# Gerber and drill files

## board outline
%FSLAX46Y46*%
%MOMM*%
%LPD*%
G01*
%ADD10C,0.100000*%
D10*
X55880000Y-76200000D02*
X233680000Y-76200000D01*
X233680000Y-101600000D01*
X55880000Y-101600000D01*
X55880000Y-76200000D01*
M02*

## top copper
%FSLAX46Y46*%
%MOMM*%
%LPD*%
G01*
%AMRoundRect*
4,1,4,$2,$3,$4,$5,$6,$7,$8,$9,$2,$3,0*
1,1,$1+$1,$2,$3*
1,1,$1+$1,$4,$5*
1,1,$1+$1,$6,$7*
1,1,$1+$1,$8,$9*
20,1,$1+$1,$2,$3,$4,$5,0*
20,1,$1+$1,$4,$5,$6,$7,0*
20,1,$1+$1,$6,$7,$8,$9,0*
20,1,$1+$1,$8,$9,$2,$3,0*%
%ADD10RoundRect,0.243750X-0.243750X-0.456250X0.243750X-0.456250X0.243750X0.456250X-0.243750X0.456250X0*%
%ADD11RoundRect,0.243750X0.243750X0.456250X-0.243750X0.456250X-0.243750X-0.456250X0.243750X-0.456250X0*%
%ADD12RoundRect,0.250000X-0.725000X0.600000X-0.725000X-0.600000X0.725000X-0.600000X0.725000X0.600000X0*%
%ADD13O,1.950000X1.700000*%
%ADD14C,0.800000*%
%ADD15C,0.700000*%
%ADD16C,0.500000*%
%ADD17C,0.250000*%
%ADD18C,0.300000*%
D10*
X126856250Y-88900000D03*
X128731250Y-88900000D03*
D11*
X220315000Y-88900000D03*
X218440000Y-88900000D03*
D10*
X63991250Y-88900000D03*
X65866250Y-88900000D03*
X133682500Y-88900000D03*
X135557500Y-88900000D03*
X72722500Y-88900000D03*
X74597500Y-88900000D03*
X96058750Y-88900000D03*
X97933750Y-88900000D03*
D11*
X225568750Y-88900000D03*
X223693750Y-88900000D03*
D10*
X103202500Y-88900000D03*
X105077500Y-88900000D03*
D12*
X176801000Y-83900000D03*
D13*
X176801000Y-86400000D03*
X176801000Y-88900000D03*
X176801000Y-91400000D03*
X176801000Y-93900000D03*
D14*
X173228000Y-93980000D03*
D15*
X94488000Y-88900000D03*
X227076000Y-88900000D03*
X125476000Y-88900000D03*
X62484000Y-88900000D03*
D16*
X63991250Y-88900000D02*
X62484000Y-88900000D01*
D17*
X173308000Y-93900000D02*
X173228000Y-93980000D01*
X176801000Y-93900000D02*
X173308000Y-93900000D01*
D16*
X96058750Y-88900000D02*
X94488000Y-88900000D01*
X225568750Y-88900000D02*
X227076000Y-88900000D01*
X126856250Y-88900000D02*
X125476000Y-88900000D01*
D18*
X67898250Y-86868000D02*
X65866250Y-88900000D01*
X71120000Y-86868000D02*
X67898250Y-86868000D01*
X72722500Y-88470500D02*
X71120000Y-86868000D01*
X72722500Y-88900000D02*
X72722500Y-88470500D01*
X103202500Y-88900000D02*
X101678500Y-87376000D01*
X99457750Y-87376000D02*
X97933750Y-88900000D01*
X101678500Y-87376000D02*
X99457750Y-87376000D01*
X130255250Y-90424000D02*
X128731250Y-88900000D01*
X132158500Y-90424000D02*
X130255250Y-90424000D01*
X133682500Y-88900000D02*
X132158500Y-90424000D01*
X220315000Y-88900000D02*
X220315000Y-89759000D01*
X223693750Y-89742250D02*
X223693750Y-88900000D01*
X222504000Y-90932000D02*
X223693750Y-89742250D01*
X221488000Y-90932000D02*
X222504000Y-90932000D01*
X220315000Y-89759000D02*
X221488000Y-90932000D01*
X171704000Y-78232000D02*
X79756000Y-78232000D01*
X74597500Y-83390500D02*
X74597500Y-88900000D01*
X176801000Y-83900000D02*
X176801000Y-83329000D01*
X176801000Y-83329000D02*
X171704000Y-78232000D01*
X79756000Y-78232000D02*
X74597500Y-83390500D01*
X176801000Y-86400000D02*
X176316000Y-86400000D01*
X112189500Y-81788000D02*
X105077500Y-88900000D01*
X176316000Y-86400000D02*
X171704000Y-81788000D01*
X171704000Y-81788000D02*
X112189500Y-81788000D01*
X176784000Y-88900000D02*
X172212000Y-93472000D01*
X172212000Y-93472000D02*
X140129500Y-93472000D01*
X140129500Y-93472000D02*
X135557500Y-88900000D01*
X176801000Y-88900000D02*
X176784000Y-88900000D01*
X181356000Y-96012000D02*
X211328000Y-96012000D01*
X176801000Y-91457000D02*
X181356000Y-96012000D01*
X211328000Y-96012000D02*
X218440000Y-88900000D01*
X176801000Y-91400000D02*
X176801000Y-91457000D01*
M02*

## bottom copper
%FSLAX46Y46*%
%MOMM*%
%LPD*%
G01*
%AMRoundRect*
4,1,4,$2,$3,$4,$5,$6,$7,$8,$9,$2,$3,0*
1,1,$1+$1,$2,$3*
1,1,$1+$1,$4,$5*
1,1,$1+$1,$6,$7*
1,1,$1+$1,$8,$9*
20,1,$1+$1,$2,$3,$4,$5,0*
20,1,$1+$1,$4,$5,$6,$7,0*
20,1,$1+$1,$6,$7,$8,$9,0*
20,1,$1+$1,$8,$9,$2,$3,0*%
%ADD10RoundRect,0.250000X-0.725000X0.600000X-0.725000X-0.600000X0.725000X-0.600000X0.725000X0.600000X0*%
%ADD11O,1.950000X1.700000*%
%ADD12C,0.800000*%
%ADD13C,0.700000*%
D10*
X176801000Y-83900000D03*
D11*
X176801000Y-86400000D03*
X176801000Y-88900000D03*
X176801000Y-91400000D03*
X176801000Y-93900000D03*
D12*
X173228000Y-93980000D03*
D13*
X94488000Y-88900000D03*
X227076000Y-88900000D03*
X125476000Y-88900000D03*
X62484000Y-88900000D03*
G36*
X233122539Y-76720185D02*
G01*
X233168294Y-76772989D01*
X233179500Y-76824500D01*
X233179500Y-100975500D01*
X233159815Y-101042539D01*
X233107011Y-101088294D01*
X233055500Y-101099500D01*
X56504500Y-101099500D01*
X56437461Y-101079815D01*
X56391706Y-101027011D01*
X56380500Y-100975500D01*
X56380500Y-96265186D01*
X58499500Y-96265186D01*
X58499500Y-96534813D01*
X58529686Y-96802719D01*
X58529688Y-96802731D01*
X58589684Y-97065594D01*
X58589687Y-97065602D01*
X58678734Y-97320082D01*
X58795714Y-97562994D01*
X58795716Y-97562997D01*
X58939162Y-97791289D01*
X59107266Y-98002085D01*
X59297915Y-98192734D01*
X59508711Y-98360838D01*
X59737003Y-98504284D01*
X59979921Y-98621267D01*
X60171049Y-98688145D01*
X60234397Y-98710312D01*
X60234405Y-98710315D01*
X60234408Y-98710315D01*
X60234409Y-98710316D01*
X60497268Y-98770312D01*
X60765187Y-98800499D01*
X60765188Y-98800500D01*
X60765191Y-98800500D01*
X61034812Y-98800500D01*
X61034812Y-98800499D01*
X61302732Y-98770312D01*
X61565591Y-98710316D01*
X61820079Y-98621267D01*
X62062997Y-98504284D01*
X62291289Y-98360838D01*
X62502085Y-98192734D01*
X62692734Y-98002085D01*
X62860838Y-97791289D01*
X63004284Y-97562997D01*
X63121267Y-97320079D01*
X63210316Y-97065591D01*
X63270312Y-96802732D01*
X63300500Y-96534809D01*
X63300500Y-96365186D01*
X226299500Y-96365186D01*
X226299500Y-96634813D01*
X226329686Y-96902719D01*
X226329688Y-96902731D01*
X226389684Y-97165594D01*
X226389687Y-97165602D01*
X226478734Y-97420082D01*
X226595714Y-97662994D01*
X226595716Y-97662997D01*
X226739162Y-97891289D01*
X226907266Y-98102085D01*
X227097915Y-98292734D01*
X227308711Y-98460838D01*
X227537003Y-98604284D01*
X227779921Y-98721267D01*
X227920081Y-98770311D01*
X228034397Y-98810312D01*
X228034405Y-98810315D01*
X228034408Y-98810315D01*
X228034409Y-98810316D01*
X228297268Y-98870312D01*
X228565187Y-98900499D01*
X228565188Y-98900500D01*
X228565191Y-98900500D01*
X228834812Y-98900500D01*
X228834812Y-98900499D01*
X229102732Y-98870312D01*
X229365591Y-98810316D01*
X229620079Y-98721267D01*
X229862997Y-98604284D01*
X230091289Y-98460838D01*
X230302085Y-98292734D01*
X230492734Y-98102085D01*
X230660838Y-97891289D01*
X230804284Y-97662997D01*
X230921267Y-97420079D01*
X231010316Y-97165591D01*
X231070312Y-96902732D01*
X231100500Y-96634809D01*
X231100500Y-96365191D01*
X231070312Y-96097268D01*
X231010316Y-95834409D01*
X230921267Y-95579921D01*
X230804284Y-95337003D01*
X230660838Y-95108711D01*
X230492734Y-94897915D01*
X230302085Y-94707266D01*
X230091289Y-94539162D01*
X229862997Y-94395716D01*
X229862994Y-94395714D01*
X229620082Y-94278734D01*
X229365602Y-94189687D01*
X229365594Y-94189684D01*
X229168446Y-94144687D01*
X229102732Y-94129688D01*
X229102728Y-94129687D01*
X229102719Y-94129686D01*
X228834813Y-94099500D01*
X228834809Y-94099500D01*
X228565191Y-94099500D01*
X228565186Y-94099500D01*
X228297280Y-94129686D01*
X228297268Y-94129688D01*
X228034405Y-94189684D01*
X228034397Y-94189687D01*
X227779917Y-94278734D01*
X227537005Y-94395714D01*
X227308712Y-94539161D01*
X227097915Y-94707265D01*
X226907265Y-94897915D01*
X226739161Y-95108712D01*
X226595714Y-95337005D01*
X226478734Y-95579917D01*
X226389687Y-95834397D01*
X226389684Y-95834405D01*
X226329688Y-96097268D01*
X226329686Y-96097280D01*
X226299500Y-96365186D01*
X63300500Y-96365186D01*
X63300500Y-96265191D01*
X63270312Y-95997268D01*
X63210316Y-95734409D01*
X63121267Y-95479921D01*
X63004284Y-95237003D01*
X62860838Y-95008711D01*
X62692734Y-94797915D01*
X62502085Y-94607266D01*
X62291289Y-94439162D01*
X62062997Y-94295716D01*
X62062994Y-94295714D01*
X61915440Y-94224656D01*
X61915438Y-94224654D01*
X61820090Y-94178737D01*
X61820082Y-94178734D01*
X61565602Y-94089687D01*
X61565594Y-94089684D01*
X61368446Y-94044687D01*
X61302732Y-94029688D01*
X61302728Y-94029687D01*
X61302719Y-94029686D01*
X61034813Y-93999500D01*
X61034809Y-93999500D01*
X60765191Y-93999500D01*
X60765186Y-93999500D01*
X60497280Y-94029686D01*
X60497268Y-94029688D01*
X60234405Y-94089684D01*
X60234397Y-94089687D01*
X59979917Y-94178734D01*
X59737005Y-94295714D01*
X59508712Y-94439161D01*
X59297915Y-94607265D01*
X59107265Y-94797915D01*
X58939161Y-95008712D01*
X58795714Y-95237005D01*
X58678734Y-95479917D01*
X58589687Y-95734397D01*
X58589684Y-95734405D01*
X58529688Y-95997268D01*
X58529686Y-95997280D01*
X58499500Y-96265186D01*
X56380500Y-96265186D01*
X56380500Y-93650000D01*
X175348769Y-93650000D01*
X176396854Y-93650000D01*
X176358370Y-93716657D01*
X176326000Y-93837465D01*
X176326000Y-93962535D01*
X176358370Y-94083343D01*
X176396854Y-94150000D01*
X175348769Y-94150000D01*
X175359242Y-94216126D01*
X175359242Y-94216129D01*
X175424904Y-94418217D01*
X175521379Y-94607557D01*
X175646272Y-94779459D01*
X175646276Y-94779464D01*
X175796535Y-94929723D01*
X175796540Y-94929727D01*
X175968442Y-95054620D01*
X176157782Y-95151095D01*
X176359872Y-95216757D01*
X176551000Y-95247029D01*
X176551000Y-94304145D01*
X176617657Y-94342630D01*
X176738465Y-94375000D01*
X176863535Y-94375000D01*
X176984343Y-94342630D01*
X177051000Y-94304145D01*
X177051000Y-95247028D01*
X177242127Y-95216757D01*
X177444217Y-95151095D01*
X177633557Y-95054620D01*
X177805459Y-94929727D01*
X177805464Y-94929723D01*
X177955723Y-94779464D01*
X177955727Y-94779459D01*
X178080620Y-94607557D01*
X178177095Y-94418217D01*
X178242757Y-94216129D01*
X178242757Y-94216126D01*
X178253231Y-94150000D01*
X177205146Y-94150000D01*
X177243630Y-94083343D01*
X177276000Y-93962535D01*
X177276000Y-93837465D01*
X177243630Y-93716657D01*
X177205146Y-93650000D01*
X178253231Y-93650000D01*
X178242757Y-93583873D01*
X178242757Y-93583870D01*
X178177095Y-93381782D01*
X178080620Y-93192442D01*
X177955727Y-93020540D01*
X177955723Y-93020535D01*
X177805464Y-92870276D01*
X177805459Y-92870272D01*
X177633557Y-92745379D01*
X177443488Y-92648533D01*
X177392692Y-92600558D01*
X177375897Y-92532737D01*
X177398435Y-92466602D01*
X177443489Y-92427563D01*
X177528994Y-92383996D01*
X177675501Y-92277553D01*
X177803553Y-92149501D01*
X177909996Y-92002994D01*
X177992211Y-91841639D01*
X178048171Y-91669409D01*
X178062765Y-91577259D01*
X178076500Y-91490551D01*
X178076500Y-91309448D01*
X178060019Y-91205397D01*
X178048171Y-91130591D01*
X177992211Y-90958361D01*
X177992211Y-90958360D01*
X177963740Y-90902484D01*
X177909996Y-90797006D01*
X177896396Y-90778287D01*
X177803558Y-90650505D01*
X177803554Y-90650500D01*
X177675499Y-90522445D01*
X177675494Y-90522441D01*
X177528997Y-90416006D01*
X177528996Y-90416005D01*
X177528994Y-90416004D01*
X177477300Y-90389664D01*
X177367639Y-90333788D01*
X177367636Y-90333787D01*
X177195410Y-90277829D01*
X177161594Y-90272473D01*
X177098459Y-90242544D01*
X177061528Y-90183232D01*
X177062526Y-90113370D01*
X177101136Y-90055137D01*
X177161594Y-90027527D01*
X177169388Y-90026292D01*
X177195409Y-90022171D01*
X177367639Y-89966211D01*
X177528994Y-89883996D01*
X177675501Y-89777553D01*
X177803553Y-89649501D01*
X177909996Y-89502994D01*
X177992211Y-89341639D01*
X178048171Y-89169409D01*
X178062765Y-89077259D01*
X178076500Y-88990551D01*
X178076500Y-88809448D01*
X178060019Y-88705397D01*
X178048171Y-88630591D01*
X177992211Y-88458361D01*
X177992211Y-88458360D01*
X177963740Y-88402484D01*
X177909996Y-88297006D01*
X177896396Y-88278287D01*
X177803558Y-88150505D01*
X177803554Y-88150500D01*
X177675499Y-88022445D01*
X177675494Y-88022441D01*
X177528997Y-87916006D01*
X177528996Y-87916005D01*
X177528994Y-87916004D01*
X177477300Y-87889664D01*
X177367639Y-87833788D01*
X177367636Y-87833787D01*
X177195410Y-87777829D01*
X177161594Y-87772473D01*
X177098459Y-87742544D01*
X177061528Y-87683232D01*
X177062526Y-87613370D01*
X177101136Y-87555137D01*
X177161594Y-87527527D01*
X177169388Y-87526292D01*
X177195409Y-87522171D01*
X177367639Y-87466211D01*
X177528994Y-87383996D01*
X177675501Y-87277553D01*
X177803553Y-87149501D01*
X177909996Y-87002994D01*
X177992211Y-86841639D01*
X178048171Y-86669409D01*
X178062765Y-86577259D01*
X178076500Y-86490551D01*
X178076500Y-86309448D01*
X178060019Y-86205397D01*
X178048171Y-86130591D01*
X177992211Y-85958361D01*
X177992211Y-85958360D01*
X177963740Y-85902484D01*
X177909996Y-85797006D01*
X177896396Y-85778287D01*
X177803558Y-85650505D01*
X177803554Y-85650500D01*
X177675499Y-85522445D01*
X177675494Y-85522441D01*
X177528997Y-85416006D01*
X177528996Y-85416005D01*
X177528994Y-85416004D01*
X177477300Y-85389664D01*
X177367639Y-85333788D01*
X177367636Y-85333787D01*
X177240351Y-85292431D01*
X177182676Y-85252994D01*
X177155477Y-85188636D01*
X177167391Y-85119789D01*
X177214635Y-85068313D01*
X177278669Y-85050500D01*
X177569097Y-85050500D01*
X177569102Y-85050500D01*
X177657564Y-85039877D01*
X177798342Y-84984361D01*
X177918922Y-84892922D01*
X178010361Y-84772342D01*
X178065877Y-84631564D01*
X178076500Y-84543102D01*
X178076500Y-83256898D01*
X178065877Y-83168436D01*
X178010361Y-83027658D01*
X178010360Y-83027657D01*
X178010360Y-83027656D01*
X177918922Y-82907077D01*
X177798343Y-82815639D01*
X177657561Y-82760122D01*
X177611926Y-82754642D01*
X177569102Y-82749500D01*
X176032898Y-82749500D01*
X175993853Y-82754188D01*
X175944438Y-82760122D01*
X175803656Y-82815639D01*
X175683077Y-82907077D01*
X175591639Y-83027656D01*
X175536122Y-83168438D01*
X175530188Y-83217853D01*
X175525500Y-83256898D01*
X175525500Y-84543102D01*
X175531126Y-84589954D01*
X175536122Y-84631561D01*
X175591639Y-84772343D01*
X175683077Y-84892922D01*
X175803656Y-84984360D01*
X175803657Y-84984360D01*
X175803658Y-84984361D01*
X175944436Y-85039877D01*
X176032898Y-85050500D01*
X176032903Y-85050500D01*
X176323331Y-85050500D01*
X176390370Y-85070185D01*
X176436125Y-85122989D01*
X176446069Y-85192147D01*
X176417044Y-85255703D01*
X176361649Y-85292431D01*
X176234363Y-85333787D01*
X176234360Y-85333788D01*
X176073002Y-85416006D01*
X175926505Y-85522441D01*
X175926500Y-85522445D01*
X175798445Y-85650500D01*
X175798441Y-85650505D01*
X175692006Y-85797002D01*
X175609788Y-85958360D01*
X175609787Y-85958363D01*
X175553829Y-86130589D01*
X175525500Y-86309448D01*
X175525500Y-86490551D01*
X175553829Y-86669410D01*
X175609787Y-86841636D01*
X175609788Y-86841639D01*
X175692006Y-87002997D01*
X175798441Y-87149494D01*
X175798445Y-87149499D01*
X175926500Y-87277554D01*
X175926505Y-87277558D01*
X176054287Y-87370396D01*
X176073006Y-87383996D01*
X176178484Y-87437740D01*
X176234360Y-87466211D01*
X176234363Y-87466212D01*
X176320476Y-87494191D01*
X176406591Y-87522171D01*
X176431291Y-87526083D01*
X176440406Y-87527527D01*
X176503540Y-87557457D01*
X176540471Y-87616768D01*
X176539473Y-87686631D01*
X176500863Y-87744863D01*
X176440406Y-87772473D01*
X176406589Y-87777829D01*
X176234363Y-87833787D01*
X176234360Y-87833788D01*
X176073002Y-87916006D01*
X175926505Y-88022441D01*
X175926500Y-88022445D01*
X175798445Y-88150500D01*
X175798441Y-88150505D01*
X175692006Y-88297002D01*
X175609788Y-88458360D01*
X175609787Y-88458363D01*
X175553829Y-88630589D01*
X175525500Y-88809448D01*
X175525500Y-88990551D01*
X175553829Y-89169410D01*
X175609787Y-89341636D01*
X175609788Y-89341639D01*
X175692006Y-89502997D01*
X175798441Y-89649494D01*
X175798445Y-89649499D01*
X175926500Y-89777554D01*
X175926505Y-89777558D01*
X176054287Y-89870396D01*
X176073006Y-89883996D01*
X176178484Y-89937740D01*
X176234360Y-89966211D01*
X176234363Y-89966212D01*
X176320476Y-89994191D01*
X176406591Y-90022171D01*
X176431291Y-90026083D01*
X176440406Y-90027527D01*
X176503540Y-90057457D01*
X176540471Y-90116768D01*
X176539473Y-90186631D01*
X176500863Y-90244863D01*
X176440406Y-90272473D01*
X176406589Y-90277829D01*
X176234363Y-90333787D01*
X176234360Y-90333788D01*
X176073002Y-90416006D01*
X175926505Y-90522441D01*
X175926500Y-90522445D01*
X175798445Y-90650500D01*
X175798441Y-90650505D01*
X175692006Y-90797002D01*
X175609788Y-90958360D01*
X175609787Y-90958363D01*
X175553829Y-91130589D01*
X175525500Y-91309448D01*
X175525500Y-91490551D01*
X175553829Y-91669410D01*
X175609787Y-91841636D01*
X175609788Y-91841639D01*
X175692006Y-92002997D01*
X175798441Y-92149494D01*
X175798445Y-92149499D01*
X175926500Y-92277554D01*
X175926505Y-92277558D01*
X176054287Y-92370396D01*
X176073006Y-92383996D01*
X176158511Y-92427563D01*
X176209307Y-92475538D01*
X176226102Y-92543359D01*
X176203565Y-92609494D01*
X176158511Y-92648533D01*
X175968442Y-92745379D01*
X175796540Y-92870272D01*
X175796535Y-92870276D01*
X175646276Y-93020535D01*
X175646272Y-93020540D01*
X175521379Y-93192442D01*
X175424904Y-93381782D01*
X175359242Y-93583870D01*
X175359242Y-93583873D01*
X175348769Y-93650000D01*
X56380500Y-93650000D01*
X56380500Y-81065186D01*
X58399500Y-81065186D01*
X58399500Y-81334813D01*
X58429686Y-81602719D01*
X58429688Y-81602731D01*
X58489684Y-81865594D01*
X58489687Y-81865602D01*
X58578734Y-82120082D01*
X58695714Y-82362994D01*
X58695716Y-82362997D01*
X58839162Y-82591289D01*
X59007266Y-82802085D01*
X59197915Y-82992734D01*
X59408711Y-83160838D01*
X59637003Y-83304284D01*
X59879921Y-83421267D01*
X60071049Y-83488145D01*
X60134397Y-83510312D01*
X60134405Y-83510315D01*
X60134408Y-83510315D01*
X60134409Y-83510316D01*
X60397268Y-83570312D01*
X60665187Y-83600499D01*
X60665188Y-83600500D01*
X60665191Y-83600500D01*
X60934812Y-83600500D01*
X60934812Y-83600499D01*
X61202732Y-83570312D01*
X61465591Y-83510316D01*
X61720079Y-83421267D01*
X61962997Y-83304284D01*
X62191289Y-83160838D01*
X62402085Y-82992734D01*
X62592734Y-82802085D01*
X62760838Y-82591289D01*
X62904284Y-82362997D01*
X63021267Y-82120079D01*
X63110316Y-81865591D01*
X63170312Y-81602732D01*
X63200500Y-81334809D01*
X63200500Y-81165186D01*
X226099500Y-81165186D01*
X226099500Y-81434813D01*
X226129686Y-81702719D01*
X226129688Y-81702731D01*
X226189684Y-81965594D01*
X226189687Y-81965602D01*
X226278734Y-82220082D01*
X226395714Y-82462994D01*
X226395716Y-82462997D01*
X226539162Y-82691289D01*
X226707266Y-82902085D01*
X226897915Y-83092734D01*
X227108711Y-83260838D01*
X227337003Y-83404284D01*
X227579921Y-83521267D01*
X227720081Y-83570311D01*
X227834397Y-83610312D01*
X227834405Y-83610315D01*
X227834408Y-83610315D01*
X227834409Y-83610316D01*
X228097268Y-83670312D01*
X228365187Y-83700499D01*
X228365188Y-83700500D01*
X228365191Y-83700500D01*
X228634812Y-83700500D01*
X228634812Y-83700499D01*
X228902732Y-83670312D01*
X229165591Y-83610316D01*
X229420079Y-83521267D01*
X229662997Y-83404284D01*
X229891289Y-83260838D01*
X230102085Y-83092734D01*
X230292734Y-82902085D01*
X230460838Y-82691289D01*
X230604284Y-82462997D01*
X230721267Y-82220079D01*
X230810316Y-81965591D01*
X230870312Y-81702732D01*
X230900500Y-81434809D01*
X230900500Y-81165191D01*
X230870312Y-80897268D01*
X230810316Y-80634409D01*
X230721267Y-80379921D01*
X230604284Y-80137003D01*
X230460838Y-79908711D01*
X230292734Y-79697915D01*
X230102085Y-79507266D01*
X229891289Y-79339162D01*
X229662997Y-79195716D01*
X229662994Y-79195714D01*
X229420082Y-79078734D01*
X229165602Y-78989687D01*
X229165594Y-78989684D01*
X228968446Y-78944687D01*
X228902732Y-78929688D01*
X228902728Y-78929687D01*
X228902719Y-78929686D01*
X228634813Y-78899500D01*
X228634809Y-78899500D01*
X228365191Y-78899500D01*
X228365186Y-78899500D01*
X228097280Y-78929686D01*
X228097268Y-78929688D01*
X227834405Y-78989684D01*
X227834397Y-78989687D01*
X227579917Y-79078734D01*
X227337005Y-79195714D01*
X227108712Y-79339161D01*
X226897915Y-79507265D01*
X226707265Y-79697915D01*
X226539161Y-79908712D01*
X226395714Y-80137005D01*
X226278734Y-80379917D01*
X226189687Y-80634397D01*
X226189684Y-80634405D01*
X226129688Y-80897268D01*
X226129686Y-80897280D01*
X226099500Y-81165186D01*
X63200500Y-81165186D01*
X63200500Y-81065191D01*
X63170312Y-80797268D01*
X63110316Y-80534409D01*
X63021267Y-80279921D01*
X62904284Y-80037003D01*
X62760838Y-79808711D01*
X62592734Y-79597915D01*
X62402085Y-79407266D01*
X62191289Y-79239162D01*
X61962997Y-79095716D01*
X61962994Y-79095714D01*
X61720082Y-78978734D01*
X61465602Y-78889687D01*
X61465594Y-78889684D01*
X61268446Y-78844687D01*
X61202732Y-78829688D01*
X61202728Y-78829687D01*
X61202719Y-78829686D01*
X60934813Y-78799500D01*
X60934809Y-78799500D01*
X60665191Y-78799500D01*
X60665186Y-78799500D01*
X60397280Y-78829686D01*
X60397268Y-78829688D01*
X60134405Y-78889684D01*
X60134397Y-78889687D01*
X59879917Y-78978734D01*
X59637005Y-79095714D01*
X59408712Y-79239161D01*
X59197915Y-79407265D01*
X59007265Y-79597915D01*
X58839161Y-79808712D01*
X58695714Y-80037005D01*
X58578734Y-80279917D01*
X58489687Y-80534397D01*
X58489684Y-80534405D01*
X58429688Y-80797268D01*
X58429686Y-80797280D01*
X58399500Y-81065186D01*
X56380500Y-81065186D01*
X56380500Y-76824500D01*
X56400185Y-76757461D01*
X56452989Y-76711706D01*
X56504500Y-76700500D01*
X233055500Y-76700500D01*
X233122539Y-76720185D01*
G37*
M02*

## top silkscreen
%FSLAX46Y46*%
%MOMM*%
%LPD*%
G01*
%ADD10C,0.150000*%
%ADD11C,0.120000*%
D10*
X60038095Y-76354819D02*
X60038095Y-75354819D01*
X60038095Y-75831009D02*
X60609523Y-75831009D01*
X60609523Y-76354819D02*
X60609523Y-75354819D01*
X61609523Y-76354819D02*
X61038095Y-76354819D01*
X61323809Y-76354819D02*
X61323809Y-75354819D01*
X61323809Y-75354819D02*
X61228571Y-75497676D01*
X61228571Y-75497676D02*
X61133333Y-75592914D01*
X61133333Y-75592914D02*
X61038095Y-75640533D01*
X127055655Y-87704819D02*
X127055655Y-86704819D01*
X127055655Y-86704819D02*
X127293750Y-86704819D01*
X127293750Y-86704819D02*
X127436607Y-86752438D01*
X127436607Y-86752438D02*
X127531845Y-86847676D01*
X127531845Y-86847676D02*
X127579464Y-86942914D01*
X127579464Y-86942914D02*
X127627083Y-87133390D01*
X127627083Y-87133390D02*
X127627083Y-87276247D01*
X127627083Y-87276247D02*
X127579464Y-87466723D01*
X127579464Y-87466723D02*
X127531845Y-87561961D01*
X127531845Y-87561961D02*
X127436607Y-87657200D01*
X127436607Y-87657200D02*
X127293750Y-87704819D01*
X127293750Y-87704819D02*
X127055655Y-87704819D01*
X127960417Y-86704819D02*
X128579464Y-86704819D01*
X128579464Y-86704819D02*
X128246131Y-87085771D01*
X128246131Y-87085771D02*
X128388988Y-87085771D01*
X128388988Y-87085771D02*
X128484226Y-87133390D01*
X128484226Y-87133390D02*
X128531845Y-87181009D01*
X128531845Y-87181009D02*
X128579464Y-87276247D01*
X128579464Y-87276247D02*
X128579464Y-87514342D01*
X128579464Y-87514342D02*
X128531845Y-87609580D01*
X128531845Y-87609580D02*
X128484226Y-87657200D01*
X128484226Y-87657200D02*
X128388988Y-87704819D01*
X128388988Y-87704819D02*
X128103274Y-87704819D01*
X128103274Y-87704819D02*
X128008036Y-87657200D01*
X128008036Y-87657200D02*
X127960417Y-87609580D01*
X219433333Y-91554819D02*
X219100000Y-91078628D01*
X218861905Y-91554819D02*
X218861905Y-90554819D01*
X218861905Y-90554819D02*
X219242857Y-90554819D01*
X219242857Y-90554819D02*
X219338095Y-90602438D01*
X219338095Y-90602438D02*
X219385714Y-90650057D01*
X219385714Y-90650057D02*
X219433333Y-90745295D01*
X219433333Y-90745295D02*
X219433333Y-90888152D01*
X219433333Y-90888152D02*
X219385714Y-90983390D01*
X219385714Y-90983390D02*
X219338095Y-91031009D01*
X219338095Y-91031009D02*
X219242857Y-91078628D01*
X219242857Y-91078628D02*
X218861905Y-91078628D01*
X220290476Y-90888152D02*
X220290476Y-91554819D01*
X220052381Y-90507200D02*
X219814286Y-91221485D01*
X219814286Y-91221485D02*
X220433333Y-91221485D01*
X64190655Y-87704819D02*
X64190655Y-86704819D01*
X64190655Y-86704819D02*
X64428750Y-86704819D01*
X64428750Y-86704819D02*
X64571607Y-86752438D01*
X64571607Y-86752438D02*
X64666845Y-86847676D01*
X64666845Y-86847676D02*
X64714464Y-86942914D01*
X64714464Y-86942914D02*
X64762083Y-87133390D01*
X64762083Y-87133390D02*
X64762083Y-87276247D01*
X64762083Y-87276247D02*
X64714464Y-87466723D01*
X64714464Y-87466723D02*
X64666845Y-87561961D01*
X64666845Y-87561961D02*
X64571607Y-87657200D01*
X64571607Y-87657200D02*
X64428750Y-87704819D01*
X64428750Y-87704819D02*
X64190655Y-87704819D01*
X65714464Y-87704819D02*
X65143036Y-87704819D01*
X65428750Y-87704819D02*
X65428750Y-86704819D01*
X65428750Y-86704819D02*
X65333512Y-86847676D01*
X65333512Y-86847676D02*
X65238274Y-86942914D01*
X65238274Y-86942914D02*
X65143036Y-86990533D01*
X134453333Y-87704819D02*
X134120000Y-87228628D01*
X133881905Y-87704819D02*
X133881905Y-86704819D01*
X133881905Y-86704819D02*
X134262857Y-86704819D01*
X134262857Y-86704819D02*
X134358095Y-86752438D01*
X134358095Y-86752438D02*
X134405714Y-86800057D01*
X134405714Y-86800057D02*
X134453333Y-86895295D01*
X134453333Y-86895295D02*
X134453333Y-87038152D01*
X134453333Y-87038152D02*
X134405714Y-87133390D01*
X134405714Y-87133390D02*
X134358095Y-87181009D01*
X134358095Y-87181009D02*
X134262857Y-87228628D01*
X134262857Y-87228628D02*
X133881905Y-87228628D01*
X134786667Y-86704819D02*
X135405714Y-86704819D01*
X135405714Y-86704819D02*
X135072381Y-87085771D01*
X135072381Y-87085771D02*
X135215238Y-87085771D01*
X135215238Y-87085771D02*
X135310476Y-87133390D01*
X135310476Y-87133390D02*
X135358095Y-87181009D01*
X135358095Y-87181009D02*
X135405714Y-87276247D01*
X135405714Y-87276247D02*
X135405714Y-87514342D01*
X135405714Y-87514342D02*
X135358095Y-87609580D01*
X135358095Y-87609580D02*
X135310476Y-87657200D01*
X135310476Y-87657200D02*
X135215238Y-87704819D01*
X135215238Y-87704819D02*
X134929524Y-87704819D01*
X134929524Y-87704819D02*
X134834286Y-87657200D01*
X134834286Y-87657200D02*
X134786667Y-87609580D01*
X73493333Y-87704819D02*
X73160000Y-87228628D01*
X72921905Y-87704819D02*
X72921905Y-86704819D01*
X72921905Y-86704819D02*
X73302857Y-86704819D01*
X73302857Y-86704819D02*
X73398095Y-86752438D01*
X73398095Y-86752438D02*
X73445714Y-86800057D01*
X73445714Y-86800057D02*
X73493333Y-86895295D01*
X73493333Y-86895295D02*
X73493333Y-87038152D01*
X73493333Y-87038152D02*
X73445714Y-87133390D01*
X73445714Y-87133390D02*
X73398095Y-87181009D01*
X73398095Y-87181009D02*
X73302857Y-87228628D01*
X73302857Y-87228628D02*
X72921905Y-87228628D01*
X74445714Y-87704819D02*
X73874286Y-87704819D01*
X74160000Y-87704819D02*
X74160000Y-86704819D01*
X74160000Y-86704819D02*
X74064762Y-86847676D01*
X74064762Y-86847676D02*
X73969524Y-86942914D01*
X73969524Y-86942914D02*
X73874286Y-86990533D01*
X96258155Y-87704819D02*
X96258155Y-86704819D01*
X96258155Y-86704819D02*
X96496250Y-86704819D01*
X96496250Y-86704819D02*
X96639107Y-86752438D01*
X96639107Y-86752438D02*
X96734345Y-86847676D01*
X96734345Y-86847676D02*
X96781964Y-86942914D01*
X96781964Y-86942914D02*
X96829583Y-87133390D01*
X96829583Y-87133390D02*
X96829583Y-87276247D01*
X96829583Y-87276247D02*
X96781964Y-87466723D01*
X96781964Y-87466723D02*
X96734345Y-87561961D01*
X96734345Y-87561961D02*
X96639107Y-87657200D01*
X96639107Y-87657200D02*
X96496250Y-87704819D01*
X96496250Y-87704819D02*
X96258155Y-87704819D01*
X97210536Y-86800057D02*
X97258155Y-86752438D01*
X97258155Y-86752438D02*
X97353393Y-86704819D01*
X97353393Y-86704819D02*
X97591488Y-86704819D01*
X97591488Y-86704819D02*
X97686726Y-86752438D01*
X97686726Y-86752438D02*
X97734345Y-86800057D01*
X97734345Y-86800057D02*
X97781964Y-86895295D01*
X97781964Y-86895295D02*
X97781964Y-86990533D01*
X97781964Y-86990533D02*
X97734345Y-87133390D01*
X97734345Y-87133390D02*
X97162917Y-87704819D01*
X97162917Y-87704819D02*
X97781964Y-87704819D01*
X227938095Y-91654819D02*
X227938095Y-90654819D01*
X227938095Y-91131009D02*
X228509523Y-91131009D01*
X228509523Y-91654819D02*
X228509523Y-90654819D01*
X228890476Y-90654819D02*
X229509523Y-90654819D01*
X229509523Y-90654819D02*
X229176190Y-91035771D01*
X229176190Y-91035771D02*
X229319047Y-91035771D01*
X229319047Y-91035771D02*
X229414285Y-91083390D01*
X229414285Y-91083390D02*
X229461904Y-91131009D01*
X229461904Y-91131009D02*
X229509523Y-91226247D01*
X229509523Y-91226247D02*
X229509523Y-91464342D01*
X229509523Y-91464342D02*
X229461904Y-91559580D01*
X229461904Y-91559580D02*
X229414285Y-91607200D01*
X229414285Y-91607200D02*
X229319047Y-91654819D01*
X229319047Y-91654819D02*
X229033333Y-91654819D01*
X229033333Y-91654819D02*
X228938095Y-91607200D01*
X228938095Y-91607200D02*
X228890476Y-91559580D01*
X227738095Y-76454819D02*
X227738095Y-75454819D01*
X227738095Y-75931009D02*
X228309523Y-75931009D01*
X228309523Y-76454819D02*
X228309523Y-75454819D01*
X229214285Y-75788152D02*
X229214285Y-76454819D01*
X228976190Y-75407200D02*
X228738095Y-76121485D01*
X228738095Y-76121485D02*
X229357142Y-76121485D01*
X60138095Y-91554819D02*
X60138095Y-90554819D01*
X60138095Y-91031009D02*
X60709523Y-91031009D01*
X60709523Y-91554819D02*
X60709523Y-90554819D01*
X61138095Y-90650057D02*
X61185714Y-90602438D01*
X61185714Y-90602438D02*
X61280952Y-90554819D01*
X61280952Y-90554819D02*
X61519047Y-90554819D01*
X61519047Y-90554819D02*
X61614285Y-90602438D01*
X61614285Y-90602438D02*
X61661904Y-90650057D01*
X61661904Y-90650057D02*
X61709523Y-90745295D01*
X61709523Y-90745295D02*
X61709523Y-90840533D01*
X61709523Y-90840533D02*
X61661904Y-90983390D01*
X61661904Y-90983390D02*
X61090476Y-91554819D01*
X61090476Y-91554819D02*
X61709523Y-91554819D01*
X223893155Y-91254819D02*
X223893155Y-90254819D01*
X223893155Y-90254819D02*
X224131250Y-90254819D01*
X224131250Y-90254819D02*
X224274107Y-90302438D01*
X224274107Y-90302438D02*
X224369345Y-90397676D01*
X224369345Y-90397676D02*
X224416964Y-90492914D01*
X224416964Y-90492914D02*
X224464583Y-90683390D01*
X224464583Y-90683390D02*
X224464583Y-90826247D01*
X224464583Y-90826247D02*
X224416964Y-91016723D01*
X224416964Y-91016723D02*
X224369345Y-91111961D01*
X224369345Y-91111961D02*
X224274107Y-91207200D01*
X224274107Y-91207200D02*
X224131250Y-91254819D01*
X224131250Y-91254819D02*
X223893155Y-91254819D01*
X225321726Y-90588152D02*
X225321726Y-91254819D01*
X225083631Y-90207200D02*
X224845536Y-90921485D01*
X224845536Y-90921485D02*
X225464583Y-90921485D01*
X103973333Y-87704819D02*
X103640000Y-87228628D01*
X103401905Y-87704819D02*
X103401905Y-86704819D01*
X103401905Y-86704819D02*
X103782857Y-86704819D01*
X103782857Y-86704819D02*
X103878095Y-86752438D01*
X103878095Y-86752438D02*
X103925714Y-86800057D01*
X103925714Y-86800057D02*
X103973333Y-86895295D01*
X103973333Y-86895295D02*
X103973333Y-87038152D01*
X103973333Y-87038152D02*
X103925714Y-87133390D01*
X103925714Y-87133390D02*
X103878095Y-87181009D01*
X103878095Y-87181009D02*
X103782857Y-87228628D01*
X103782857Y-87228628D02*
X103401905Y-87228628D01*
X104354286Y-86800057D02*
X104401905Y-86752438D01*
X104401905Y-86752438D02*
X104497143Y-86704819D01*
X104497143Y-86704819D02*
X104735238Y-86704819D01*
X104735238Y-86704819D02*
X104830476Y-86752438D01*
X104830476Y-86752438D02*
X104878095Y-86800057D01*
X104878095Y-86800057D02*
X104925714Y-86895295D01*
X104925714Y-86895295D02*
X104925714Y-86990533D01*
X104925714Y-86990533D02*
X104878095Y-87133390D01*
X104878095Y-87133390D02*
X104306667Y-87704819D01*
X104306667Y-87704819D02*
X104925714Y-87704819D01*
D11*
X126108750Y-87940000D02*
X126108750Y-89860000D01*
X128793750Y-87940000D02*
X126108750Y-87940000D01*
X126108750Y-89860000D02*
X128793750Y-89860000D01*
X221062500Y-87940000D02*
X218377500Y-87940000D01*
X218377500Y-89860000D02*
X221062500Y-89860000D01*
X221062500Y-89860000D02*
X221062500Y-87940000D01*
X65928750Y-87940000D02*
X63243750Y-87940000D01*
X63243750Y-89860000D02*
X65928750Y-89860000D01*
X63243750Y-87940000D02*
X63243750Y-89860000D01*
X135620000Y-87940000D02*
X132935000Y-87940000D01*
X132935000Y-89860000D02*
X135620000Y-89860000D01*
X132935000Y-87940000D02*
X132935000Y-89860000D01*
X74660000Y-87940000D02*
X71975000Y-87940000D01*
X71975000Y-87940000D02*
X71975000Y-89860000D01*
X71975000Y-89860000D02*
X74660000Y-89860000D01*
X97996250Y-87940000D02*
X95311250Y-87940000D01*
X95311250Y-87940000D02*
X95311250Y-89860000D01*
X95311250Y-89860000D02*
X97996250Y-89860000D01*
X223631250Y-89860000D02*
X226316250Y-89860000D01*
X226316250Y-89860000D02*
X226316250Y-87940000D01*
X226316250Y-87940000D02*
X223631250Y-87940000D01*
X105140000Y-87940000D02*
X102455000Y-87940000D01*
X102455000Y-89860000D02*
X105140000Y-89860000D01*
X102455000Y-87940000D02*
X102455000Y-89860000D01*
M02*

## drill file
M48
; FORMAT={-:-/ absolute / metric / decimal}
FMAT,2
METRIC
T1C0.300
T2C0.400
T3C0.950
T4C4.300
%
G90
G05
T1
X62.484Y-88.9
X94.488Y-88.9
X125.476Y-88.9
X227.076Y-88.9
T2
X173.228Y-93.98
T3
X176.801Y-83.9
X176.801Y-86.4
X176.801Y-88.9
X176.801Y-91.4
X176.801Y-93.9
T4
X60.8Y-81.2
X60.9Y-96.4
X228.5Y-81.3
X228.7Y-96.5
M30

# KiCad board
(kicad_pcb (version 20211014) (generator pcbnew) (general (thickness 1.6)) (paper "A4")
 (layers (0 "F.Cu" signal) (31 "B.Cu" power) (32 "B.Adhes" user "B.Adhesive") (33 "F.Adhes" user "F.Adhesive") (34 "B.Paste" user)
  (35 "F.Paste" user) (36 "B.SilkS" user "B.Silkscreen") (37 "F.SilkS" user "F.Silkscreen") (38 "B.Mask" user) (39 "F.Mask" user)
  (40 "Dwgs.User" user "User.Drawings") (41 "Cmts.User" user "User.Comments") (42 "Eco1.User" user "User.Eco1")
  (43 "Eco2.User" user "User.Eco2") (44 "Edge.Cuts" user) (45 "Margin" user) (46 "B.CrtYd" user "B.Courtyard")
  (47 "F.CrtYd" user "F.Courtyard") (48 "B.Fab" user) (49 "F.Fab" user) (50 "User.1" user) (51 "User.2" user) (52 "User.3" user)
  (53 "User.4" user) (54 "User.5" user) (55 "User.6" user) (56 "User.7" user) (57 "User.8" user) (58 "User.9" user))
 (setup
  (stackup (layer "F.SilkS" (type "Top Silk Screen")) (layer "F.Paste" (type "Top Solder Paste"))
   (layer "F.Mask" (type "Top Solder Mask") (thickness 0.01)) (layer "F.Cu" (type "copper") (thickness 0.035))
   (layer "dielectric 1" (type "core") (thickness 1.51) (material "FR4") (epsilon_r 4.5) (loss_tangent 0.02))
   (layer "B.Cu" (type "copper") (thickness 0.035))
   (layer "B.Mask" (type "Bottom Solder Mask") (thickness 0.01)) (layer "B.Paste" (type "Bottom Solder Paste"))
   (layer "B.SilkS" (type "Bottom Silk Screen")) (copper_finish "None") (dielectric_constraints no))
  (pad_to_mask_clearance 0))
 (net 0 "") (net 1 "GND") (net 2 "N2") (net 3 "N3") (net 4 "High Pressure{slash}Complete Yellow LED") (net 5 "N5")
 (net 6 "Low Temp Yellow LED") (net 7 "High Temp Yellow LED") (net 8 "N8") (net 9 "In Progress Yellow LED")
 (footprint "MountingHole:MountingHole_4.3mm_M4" (layer "F.Cu") (at 60.8 81.2)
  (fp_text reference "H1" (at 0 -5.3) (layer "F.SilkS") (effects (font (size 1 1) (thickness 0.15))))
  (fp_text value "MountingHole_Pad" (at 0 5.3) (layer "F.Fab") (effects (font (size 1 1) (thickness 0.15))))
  (pad "" np_thru_hole circle locked (at 0 0) (size 4.3 4.3) (drill 4.3) (layers *.Cu *.Mask)))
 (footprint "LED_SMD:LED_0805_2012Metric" (layer "F.Cu") (at 127.79375 88.9)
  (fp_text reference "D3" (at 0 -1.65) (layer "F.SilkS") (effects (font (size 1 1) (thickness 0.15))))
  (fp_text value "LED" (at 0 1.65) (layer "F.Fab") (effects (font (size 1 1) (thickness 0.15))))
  (fp_line (start -1.685 -0.96) (end -1.685 0.96) (layer "F.SilkS") (width 0.12))
  (fp_line (start 1 -0.96) (end -1.685 -0.96) (layer "F.SilkS") (width 0.12))
  (fp_line (start -1.685 0.96) (end 1 0.96) (layer "F.SilkS") (width 0.12))
  (pad "1" smd roundrect locked (at -0.9375 0) (size 0.975 1.4) (layers "F.Cu" "F.Paste" "F.Mask") (roundrect_rratio 0.25) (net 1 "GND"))
  (pad "2" smd roundrect locked (at 0.9375 0) (size 0.975 1.4) (layers "F.Cu" "F.Paste" "F.Mask") (roundrect_rratio 0.25) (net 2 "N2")))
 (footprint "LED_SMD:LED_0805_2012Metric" (layer "F.Cu") (at 219.3775 88.9 180)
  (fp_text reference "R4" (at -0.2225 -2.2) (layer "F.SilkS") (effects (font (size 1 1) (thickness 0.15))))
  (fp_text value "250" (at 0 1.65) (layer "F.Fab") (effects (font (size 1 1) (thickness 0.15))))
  (fp_line (start -1.685 0.96) (end 1 0.96) (layer "F.SilkS") (width 0.12))
  (fp_line (start 1 -0.96) (end -1.685 -0.96) (layer "F.SilkS") (width 0.12))
  (fp_line (start -1.685 -0.96) (end -1.685 0.96) (layer "F.SilkS") (width 0.12))
  (pad "1" smd roundrect locked (at -0.9375 0 180) (size 0.975 1.4) (layers "F.Cu" "F.Paste" "F.Mask") (roundrect_rratio 0.25) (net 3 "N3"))
  (pad "2" smd roundrect locked (at 0.9375 0 180) (size 0.975 1.4) (layers "F.Cu" "F.Paste" "F.Mask") (roundrect_rratio 0.25)
   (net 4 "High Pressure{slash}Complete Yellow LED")))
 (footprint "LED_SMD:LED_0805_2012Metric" (layer "F.Cu") (at 64.92875 88.9)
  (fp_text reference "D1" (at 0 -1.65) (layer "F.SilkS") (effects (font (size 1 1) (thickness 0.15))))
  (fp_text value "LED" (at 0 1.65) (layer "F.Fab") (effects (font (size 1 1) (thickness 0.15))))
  (fp_line (start 1 -0.96) (end -1.685 -0.96) (layer "F.SilkS") (width 0.12))
  (fp_line (start -1.685 0.96) (end 1 0.96) (layer "F.SilkS") (width 0.12))
  (fp_line (start -1.685 -0.96) (end -1.685 0.96) (layer "F.SilkS") (width 0.12))
  (pad "1" smd roundrect locked (at -0.9375 0) (size 0.975 1.4) (layers "F.Cu" "F.Paste" "F.Mask") (roundrect_rratio 0.25) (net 1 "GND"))
  (pad "2" smd roundrect locked (at 0.9375 0) (size 0.975 1.4) (layers "F.Cu" "F.Paste" "F.Mask") (roundrect_rratio 0.25) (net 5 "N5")))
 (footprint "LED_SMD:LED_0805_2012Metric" (layer "F.Cu") (at 134.62 88.9)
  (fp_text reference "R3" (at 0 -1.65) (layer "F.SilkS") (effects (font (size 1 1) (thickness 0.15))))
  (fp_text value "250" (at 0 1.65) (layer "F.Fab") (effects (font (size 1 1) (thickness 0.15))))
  (fp_line (start 1 -0.96) (end -1.685 -0.96) (layer "F.SilkS") (width 0.12))
  (fp_line (start -1.685 0.96) (end 1 0.96) (layer "F.SilkS") (width 0.12))
  (fp_line (start -1.685 -0.96) (end -1.685 0.96) (layer "F.SilkS") (width 0.12))
  (pad "1" smd roundrect locked (at -0.9375 0) (size 0.975 1.4) (layers "F.Cu" "F.Paste" "F.Mask") (roundrect_rratio 0.25) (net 2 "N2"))
  (pad "2" smd roundrect locked (at 0.9375 0) (size 0.975 1.4) (layers "F.Cu" "F.Paste" "F.Mask") (roundrect_rratio 0.25)
   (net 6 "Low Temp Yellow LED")))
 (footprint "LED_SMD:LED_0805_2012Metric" (layer "F.Cu") (at 73.66 88.9)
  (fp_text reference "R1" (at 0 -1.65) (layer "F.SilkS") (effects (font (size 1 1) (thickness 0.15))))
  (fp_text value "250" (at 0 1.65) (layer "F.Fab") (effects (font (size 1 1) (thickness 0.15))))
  (fp_line (start 1 -0.96) (end -1.685 -0.96) (layer "F.SilkS") (width 0.12))
  (fp_line (start -1.685 -0.96) (end -1.685 0.96) (layer "F.SilkS") (width 0.12))
  (fp_line (start -1.685 0.96) (end 1 0.96) (layer "F.SilkS") (width 0.12))
  (pad "1" smd roundrect locked (at -0.9375 0) (size 0.975 1.4) (layers "F.Cu" "F.Paste" "F.Mask") (roundrect_rratio 0.25) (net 5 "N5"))
  (pad "2" smd roundrect locked (at 0.9375 0) (size 0.975 1.4) (layers "F.Cu" "F.Paste" "F.Mask") (roundrect_rratio 0.25)
   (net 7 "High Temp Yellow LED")))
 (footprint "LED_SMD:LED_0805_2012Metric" (layer "F.Cu") (at 96.99625 88.9)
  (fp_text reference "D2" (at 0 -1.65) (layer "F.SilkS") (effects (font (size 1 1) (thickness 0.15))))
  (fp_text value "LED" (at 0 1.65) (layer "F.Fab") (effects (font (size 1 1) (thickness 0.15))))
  (fp_line (start 1 -0.96) (end -1.685 -0.96) (layer "F.SilkS") (width 0.12))
  (fp_line (start -1.685 -0.96) (end -1.685 0.96) (layer "F.SilkS") (width 0.12))
  (fp_line (start -1.685 0.96) (end 1 0.96) (layer "F.SilkS") (width 0.12))
  (pad "1" smd roundrect locked (at -0.9375 0) (size 0.975 1.4) (layers "F.Cu" "F.Paste" "F.Mask") (roundrect_rratio 0.25) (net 1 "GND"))
  (pad "2" smd roundrect locked (at 0.9375 0) (size 0.975 1.4) (layers "F.Cu" "F.Paste" "F.Mask") (roundrect_rratio 0.25) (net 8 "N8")))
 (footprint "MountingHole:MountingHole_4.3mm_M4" (layer "F.Cu") (at 228.7 96.5)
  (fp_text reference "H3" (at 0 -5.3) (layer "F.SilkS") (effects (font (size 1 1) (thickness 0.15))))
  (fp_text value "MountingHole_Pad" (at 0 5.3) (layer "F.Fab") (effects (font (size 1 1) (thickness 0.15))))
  (pad "" np_thru_hole circle locked (at 0 0) (size 4.3 4.3) (drill 4.3) (layers *.Cu *.Mask)))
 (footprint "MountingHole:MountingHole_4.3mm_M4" (layer "F.Cu") (at 228.5 81.3)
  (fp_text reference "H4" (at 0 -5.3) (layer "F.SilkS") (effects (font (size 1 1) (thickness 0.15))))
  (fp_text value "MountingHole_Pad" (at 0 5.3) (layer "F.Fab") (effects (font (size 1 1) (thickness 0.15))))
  (pad "" np_thru_hole circle locked (at 0 0) (size 4.3 4.3) (drill 4.3) (layers *.Cu *.Mask)))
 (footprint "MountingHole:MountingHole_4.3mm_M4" (layer "F.Cu") (at 60.9 96.4)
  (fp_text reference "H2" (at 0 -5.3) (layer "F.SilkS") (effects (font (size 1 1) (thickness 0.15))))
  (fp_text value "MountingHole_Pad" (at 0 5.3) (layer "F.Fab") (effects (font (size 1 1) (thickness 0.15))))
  (pad "" np_thru_hole circle locked (at 0 0) (size 4.3 4.3) (drill 4.3) (layers *.Cu *.Mask)))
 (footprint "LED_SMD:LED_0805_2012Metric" (layer "F.Cu") (at 224.63125 88.9 180)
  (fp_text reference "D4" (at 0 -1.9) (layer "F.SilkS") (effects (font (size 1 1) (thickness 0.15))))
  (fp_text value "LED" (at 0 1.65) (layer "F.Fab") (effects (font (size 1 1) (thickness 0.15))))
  (fp_line (start 1 -0.96) (end -1.685 -0.96) (layer "F.SilkS") (width 0.12))
  (fp_line (start -1.685 -0.96) (end -1.685 0.96) (layer "F.SilkS") (width 0.12))
  (fp_line (start -1.685 0.96) (end 1 0.96) (layer "F.SilkS") (width 0.12))
  (pad "1" smd roundrect locked (at -0.9375 0 180) (size 0.975 1.4) (layers "F.Cu" "F.Paste" "F.Mask") (roundrect_rratio 0.25) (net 1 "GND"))
  (pad "2" smd roundrect locked (at 0.9375 0 180) (size 0.975 1.4) (layers "F.Cu" "F.Paste" "F.Mask") (roundrect_rratio 0.25) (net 3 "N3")))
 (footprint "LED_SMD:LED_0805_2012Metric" (layer "F.Cu") (at 104.14 88.9)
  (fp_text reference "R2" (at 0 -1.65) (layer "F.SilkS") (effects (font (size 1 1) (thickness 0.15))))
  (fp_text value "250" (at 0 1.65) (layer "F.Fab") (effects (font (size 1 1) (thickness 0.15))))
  (fp_line (start 1 -0.96) (end -1.685 -0.96) (layer "F.SilkS") (width 0.12))
  (fp_line (start -1.685 0.96) (end 1 0.96) (layer "F.SilkS") (width 0.12))
  (fp_line (start -1.685 -0.96) (end -1.685 0.96) (layer "F.SilkS") (width 0.12))
  (pad "1" smd roundrect locked (at -0.9375 0) (size 0.975 1.4) (layers "F.Cu" "F.Paste" "F.Mask") (roundrect_rratio 0.25) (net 8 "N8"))
  (pad "2" smd roundrect locked (at 0.9375 0) (size 0.975 1.4) (layers "F.Cu" "F.Paste" "F.Mask") (roundrect_rratio 0.25)
   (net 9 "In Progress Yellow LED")))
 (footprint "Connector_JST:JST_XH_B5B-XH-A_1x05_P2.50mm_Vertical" (layer "B.Cu") (at 176.801 83.9 -90)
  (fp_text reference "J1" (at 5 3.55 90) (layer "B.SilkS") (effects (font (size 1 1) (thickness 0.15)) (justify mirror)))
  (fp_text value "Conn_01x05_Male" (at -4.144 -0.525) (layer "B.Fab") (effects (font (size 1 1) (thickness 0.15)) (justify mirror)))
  (pad "1" thru_hole roundrect locked (at 0 0 270) (size 1.7 1.95) (drill 0.95) (layers *.Cu *.Mask) (roundrect_rratio 0.147059)
   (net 7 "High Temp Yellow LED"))
  (pad "2" thru_hole oval locked (at 2.5 0 270) (size 1.7 1.95) (drill 0.95) (layers *.Cu *.Mask) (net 9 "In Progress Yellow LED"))
  (pad "3" thru_hole oval locked (at 5 0 270) (size 1.7 1.95) (drill 0.95) (layers *.Cu *.Mask) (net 6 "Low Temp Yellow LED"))
  (pad "4" thru_hole oval locked (at 7.5 0 270) (size 1.7 1.95) (drill 0.95) (layers *.Cu *.Mask)
   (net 4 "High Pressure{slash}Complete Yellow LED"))
  (pad "5" thru_hole oval locked (at 10 0 270) (size 1.7 1.95) (drill 0.95) (layers *.Cu *.Mask) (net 1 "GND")))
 (gr_rect (start 55.88 76.2) (end 233.68 101.6) (layer "Edge.Cuts") (width 0.1) (fill none))
 (segment (start 63.99125 88.9) (end 62.484 88.9) (width 0.5) (layer "F.Cu") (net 1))
 (segment (start 173.308 93.9) (end 173.228 93.98) (width 0.25) (layer "F.Cu") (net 1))
 (segment (start 176.801 93.9) (end 173.308 93.9) (width 0.25) (layer "F.Cu") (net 1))
 (segment (start 96.05875 88.9) (end 94.488 88.9) (width 0.5) (layer "F.Cu") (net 1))
 (segment (start 225.56875 88.9) (end 227.076 88.9) (width 0.5) (layer "F.Cu") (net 1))
 (segment (start 126.85625 88.9) (end 125.476 88.9) (width 0.5) (layer "F.Cu") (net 1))
 (via (at 173.228 93.98) (size 0.8) (drill 0.4) (layers "F.Cu" "B.Cu") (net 1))
 (via (at 94.488 88.9) (size 0.7) (drill 0.3) (layers "F.Cu" "B.Cu") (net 1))
 (via (at 227.076 88.9) (size 0.7) (drill 0.3) (layers "F.Cu" "B.Cu") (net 1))
 (via (at 125.476 88.9) (size 0.7) (drill 0.3) (layers "F.Cu" "B.Cu") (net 1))
 (via (at 62.484 88.9) (size 0.7) (drill 0.3) (layers "F.Cu" "B.Cu") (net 1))
 (segment (start 67.89825 86.868) (end 65.86625 88.9) (width 0.3) (layer "F.Cu") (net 5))
 (segment (start 71.12 86.868) (end 67.89825 86.868) (width 0.3) (layer "F.Cu") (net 5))
 (segment (start 72.7225 88.4705) (end 71.12 86.868) (width 0.3) (layer "F.Cu") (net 5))
 (segment (start 72.7225 88.9) (end 72.7225 88.4705) (width 0.3) (layer "F.Cu") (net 5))
 (segment (start 103.2025 88.9) (end 101.6785 87.376) (width 0.3) (layer "F.Cu") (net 8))
 (segment (start 99.45775 87.376) (end 97.93375 88.9) (width 0.3) (layer "F.Cu") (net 8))
 (segment (start 101.6785 87.376) (end 99.45775 87.376) (width 0.3) (layer "F.Cu") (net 8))
 (segment (start 130.25525 90.424) (end 128.73125 88.9) (width 0.3) (layer "F.Cu") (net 2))
 (segment (start 132.1585 90.424) (end 130.25525 90.424) (width 0.3) (layer "F.Cu") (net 2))
 (segment (start 133.6825 88.9) (end 132.1585 90.424) (width 0.3) (layer "F.Cu") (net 2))
 (segment (start 220.315 88.9) (end 220.315 89.759) (width 0.3) (layer "F.Cu") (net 3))
 (segment (start 223.69375 89.74225) (end 223.69375 88.9) (width 0.3) (layer "F.Cu") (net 3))
 (segment (start 222.504 90.932) (end 223.69375 89.74225) (width 0.3) (layer "F.Cu") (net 3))
 (segment (start 221.488 90.932) (end 222.504 90.932) (width 0.3) (layer "F.Cu") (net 3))
 (segment (start 220.315 89.759) (end 221.488 90.932) (width 0.3) (layer "F.Cu") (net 3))
 (segment (start 171.704 78.232) (end 79.756 78.232) (width 0.3) (layer "F.Cu") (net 7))
 (segment (start 74.5975 83.3905) (end 74.5975 88.9) (width 0.3) (layer "F.Cu") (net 7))
 (segment (start 176.801 83.9) (end 176.801 83.329) (width 0.3) (layer "F.Cu") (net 7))
 (segment (start 176.801 83.329) (end 171.704 78.232) (width 0.3) (layer "F.Cu") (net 7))
 (segment (start 79.756 78.232) (end 74.5975 83.3905) (width 0.3) (layer "F.Cu") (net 7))
 (segment (start 176.801 86.4) (end 176.316 86.4) (width 0.3) (layer "F.Cu") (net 9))
 (segment (start 112.1895 81.788) (end 105.0775 88.9) (width 0.3) (layer "F.Cu") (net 9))
 (segment (start 176.316 86.4) (end 171.704 81.788) (width 0.3) (layer "F.Cu") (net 9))
 (segment (start 171.704 81.788) (end 112.1895 81.788) (width 0.3) (layer "F.Cu") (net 9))
 (segment (start 176.784 88.9) (end 172.212 93.472) (width 0.3) (layer "F.Cu") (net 6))
 (segment (start 172.212 93.472) (end 140.1295 93.472) (width 0.3) (layer "F.Cu") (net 6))
 (segment (start 140.1295 93.472) (end 135.5575 88.9) (width 0.3) (layer "F.Cu") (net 6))
 (segment (start 176.801 88.9) (end 176.784 88.9) (width 0.3) (layer "F.Cu") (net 6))
 (segment (start 181.356 96.012) (end 211.328 96.012) (width 0.3) (layer "F.Cu") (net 4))
 (segment (start 176.801 91.457) (end 181.356 96.012) (width 0.3) (layer "F.Cu") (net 4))
 (segment (start 211.328 96.012) (end 218.44 88.9) (width 0.3) (layer "F.Cu") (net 4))
 (segment (start 176.801 91.4) (end 176.801 91.457) (width 0.3) (layer "F.Cu") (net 4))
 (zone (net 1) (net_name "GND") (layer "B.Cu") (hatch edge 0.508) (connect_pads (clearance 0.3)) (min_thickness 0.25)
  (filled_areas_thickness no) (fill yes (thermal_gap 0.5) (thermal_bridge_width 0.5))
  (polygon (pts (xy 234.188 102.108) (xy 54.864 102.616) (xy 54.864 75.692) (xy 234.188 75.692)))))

